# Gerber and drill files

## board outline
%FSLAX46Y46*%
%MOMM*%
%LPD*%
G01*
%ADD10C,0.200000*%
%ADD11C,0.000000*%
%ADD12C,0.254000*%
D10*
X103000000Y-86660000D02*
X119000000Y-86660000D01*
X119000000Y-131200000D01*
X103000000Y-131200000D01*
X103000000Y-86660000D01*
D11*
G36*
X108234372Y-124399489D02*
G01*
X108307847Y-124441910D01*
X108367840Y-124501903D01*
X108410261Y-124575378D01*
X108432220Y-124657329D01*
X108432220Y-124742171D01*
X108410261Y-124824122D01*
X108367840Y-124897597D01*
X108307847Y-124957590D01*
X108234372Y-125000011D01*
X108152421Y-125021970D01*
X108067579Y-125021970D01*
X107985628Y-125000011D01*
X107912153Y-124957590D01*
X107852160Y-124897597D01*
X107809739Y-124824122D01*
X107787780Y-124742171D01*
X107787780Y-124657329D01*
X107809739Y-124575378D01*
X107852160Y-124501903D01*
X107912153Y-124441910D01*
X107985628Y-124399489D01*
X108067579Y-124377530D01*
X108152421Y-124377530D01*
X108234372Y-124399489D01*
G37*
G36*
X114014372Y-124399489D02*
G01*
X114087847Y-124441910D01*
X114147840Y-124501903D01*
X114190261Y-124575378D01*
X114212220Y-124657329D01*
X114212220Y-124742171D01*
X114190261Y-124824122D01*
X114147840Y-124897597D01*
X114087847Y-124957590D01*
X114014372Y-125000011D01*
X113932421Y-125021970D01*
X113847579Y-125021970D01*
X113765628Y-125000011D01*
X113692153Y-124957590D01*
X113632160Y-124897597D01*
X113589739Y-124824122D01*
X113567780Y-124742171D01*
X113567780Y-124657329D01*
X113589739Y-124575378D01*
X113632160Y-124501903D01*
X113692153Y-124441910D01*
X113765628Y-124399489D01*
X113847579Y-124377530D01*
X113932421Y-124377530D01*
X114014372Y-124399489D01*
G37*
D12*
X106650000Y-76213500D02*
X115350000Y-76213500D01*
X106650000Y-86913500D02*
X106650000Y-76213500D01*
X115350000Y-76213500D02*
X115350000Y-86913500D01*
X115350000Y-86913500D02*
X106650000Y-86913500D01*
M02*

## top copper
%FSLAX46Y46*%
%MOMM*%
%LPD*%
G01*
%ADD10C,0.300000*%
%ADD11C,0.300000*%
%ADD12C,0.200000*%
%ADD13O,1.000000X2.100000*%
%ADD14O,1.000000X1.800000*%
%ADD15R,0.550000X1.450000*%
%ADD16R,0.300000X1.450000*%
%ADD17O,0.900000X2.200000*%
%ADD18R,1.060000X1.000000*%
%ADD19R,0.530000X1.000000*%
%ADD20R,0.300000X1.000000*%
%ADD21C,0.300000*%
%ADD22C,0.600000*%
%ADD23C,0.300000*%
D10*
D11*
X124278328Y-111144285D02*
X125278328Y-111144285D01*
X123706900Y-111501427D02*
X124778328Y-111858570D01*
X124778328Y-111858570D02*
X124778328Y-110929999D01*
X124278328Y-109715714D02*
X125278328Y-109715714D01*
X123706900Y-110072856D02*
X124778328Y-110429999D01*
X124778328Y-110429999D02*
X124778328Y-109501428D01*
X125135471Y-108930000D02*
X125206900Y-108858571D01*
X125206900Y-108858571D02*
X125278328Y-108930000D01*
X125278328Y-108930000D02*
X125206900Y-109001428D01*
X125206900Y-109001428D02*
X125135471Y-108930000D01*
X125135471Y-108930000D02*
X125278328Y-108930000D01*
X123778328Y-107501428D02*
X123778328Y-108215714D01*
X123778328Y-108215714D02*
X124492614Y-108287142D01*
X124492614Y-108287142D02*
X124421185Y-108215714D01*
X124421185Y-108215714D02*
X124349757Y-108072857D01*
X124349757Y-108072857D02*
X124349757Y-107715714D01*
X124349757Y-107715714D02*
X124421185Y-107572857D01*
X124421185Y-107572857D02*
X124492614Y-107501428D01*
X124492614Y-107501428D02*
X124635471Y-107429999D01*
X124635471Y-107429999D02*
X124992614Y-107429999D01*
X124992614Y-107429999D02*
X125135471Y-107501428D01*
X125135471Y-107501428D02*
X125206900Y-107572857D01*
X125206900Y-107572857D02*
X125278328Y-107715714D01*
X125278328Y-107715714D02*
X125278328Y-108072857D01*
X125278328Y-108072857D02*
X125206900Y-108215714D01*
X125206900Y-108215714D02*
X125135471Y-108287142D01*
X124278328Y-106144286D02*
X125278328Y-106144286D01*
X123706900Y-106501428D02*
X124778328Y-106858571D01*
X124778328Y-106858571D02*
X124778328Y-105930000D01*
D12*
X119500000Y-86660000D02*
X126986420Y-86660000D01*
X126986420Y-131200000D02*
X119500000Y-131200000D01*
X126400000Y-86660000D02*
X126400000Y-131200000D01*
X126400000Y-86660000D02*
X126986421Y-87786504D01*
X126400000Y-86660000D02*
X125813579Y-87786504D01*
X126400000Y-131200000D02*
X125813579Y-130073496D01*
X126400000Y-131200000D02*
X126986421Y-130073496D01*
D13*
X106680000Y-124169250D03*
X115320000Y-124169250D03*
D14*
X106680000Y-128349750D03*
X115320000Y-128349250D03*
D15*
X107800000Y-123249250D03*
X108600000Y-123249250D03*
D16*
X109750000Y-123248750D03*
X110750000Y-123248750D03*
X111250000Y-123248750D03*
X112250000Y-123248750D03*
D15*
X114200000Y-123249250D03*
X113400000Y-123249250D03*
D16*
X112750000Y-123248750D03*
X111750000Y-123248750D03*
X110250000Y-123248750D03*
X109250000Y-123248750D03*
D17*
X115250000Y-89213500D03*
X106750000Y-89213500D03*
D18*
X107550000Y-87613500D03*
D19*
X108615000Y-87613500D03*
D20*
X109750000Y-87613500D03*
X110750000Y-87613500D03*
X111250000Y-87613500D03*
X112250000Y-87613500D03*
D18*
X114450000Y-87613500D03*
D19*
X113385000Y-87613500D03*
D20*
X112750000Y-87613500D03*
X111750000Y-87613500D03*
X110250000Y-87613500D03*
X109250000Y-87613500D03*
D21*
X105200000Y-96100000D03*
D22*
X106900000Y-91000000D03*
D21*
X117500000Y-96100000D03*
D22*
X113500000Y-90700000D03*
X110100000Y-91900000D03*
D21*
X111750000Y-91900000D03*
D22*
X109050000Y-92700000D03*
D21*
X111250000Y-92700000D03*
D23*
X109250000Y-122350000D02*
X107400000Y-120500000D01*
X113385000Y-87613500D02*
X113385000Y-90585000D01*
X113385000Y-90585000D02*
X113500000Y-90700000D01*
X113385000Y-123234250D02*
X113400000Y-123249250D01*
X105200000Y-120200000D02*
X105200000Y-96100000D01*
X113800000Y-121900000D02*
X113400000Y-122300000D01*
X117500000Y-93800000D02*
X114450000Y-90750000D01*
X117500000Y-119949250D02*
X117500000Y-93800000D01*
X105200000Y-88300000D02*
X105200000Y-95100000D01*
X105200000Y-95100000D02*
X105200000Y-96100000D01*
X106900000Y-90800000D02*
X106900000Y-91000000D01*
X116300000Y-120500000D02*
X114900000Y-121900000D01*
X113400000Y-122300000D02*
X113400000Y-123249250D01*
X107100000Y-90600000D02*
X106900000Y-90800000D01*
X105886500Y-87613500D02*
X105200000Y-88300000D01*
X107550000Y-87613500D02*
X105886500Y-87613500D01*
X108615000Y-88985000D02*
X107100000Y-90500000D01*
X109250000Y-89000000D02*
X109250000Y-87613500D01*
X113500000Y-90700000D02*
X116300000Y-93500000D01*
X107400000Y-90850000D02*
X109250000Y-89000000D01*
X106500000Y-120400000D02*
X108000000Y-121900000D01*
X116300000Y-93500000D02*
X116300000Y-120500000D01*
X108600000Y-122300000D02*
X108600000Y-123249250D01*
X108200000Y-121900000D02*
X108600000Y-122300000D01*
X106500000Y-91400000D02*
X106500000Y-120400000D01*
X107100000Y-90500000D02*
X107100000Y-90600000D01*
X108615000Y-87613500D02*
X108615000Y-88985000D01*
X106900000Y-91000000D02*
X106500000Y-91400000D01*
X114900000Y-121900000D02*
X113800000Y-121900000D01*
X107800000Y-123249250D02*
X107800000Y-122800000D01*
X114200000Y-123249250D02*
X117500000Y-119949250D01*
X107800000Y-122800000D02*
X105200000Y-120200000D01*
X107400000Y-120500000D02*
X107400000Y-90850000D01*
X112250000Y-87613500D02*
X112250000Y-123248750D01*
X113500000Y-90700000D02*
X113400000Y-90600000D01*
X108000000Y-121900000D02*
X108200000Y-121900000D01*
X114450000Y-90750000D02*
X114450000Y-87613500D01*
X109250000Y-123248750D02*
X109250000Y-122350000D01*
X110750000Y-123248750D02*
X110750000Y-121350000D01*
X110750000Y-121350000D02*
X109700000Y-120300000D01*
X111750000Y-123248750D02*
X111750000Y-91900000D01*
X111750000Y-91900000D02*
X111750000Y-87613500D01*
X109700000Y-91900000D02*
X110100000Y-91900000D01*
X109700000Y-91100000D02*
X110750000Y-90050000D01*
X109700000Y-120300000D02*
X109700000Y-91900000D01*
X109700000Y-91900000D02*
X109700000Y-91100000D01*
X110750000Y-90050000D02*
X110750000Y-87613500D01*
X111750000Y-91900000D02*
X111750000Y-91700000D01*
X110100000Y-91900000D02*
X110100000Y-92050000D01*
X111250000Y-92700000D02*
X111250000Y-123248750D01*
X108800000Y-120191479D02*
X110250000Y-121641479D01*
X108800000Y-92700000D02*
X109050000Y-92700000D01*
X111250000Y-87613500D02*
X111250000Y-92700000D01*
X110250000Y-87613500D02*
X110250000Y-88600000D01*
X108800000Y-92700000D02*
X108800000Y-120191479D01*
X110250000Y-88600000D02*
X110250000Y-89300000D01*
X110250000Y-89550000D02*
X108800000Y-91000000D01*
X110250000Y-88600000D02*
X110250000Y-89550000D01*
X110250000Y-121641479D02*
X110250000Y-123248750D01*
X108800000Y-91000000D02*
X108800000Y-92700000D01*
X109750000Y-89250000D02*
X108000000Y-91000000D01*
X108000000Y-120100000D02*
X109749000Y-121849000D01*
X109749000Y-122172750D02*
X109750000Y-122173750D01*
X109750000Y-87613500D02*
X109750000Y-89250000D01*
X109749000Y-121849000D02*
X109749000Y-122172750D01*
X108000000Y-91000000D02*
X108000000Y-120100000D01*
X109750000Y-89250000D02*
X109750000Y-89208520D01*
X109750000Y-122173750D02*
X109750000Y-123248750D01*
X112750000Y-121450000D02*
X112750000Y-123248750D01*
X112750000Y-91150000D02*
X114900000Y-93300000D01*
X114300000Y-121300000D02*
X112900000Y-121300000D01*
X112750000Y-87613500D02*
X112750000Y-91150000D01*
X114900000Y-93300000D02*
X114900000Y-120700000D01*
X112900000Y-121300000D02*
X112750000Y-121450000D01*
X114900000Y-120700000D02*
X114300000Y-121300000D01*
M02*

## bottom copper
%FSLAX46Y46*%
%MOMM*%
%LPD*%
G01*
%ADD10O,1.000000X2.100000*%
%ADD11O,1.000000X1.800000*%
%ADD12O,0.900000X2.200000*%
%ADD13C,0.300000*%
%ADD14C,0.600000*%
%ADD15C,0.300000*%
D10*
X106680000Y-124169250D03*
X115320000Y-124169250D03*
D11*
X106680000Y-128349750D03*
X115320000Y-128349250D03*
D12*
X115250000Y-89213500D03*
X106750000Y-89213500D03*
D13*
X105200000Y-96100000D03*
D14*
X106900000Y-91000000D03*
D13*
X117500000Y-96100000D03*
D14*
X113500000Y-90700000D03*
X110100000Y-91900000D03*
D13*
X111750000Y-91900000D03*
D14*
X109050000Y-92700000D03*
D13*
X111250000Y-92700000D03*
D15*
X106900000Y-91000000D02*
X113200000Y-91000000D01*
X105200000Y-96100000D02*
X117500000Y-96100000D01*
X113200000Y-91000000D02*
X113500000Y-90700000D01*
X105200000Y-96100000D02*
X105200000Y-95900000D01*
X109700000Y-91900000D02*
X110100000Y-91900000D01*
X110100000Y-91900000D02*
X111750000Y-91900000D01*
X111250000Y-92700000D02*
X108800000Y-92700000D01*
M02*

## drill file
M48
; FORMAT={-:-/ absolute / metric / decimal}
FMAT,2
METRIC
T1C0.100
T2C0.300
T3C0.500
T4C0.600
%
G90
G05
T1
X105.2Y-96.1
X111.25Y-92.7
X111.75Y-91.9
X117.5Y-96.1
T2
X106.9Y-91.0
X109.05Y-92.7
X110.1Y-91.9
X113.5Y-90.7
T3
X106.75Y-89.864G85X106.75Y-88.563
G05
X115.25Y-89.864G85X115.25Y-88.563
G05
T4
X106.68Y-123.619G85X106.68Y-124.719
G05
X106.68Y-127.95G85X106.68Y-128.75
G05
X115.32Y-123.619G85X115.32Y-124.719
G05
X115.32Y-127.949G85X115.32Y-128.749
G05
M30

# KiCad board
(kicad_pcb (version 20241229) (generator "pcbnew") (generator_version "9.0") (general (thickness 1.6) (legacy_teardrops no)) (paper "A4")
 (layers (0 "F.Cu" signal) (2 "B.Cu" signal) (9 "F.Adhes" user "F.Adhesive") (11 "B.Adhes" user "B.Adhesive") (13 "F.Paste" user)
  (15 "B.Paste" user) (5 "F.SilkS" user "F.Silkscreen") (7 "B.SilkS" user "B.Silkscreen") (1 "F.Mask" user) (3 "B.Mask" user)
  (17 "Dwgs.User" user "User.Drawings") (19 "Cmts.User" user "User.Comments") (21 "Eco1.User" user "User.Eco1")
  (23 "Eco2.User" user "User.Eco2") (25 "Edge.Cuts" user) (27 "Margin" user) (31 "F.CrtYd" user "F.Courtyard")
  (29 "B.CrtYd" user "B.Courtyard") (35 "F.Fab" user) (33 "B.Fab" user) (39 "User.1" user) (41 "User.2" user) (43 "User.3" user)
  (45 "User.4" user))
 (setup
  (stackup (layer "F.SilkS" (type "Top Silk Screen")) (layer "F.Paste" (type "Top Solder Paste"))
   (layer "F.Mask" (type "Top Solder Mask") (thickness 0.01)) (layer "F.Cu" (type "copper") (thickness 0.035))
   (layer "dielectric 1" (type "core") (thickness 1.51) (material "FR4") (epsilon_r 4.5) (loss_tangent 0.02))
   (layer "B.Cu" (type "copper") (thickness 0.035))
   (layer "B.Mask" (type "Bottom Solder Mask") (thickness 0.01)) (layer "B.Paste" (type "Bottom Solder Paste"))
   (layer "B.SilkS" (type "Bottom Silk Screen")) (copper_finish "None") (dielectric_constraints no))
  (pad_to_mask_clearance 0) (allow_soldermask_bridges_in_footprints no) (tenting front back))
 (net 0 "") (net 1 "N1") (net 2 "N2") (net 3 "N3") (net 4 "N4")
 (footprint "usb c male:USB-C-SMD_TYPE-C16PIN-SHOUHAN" (layer "F.Cu") (at 111 125.79925)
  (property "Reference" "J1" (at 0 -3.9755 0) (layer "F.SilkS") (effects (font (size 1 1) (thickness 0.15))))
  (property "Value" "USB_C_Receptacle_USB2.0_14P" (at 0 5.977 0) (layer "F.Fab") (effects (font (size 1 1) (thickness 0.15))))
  (fp_poly
   (pts (xy -2.56778 -1.141921) (xy -2.589739 -1.223872) (xy -2.63216 -1.297347) (xy -2.692153 -1.35734) (xy -2.765628 -1.399761)
    (xy -2.847579 -1.42172) (xy -2.932421 -1.42172) (xy -3.014372 -1.399761) (xy -3.087847 -1.35734) (xy -3.14784 -1.297347)
    (xy -3.190261 -1.223872) (xy -3.21222 -1.141921) (xy -3.21222 -1.057079) (xy -3.190261 -0.975128) (xy -3.14784 -0.901653)
    (xy -3.087847 -0.84166) (xy -3.014372 -0.799239) (xy -2.932421 -0.77728) (xy -2.847579 -0.77728) (xy -2.765628 -0.799239)
    (xy -2.692153 -0.84166) (xy -2.63216 -0.901653) (xy -2.589739 -0.975128) (xy -2.56778 -1.057079))
   (stroke (width 0) (type default)) (fill yes) (layer "Edge.Cuts"))
  (fp_poly
   (pts (xy 3.21222 -1.141921) (xy 3.190261 -1.223872) (xy 3.14784 -1.297347) (xy 3.087847 -1.35734) (xy 3.014372 -1.399761)
    (xy 2.932421 -1.42172) (xy 2.847579 -1.42172) (xy 2.765628 -1.399761) (xy 2.692153 -1.35734) (xy 2.63216 -1.297347)
    (xy 2.589739 -1.223872) (xy 2.56778 -1.141921) (xy 2.56778 -1.057079) (xy 2.589739 -0.975128) (xy 2.63216 -0.901653)
    (xy 2.692153 -0.84166) (xy 2.765628 -0.799239) (xy 2.847579 -0.77728) (xy 2.932421 -0.77728) (xy 3.014372 -0.799239)
    (xy 3.087847 -0.84166) (xy 3.14784 -0.901653) (xy 3.190261 -0.975128) (xy 3.21222 -1.057079))
   (stroke (width 0) (type default)) (fill yes) (layer "Edge.Cuts"))
  (pad "1" thru_hole oval (at -4.32 -1.63) (size 1 2.1) (drill oval 0.6 1.7) (layers "*.Cu" "*.Mask") (remove_unused_layers no))
  (pad "2" thru_hole oval (at 4.32 -1.63) (size 1 2.1) (drill oval 0.6 1.7) (layers "*.Cu" "*.Mask") (remove_unused_layers no))
  (pad "3" thru_hole oval (at -4.32 2.5505) (size 1 1.8) (drill oval 0.6 1.4) (layers "*.Cu" "*.Mask") (remove_unused_layers no))
  (pad "4" thru_hole oval (at 4.32 2.55) (size 1 1.8) (drill oval 0.6 1.4) (layers "*.Cu" "*.Mask") (remove_unused_layers no))
  (pad "A1B12" smd rect (at -3.2 -2.55) (size 0.55 1.45) (layers "F.Cu" "F.Mask" "F.Paste"))
  (pad "A4B9" smd rect (at -2.4 -2.55) (size 0.55 1.45) (layers "F.Cu" "F.Mask" "F.Paste"))
  (pad "A5" smd rect (at -1.25 -2.5505) (size 0.3 1.45) (layers "F.Cu" "F.Mask" "F.Paste") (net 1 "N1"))
  (pad "A6" smd rect (at -0.25 -2.5505) (size 0.3 1.45) (layers "F.Cu" "F.Mask" "F.Paste") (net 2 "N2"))
  (pad "A7" smd rect (at 0.25 -2.5505) (size 0.3 1.45) (layers "F.Cu" "F.Mask" "F.Paste") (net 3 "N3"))
  (pad "A8" smd rect (at 1.25 -2.5505) (size 0.3 1.45) (layers "F.Cu" "F.Mask" "F.Paste"))
  (pad "B1A12" smd rect (at 3.2 -2.55) (size 0.55 1.45) (layers "F.Cu" "F.Mask" "F.Paste"))
  (pad "B4A9" smd rect (at 2.4 -2.55) (size 0.55 1.45) (layers "F.Cu" "F.Mask" "F.Paste"))
  (pad "B5" smd rect (at 1.75 -2.5505) (size 0.3 1.45) (layers "F.Cu" "F.Mask" "F.Paste") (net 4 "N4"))
  (pad "B6" smd rect (at 0.75 -2.5505) (size 0.3 1.45) (layers "F.Cu" "F.Mask" "F.Paste") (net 2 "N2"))
  (pad "B7" smd rect (at -0.75 -2.5505) (size 0.3 1.45) (layers "F.Cu" "F.Mask" "F.Paste") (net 3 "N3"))
  (pad "B8" smd rect (at -1.75 -2.5505) (size 0.3 1.45) (layers "F.Cu" "F.Mask" "F.Paste")))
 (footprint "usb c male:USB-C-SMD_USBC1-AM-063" (layer "F.Cu") (at 111 88.4135 180)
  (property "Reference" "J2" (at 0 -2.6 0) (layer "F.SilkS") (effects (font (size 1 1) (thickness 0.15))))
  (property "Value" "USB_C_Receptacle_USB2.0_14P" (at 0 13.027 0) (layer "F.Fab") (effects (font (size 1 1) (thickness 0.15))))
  (fp_line (start 4.35 12.2) (end -4.35 12.2) (stroke (width 0.254) (type default)) (layer "Edge.Cuts"))
  (fp_line (start 4.35 1.5) (end 4.35 12.2) (stroke (width 0.254) (type default)) (layer "Edge.Cuts"))
  (fp_line (start -4.35 12.2) (end -4.35 1.5) (stroke (width 0.254) (type default)) (layer "Edge.Cuts"))
  (fp_line (start -4.35 1.5) (end 4.35 1.5) (stroke (width 0.254) (type default)) (layer "Edge.Cuts"))
  (pad "1" thru_hole oval (at -4.25 -0.8 180) (size 0.9 2.2) (drill oval 0.5 1.8) (layers "*.Cu" "*.Mask") (remove_unused_layers no))
  (pad "2" thru_hole oval (at 4.25 -0.8 180) (size 0.9 2.2) (drill oval 0.5 1.8) (layers "*.Cu" "*.Mask") (remove_unused_layers no))
  (pad "A1B12" smd rect (at 3.45 0.8) (size 1.06 1) (layers "F.Cu" "F.Mask" "F.Paste"))
  (pad "A4B9" smd rect (at 2.385 0.8) (size 0.53 1) (layers "F.Cu" "F.Mask" "F.Paste"))
  (pad "A5" smd rect (at 1.25 0.8) (size 0.3 1) (layers "F.Cu" "F.Mask" "F.Paste") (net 1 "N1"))
  (pad "A6" smd rect (at 0.25 0.8 180) (size 0.3 1) (layers "F.Cu" "F.Mask" "F.Paste") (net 2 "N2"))
  (pad "A7" smd rect (at -0.25 0.8) (size 0.3 1) (layers "F.Cu" "F.Mask" "F.Paste") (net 3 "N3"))
  (pad "A8" smd rect (at -1.25 0.8) (size 0.3 1) (layers "F.Cu" "F.Mask" "F.Paste"))
  (pad "B1A12" smd rect (at -3.45 0.8) (size 1.06 1) (layers "F.Cu" "F.Mask" "F.Paste"))
  (pad "B4A9" smd rect (at -2.385 0.8) (size 0.53 1) (layers "F.Cu" "F.Mask" "F.Paste"))
  (pad "B5" smd rect (at -1.75 0.8) (size 0.3 1) (layers "F.Cu" "F.Mask" "F.Paste") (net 4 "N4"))
  (pad "B6" smd rect (at -0.75 0.8 180) (size 0.3 1) (layers "F.Cu" "F.Mask" "F.Paste") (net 2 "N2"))
  (pad "B7" smd rect (at 0.75 0.8) (size 0.3 1) (layers "F.Cu" "F.Mask" "F.Paste") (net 3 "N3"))
  (pad "B8" smd rect (at 1.75 0.8) (size 0.3 1) (layers "F.Cu" "F.Mask" "F.Paste")))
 (gr_rect (start 103 86.66) (end 119 131.2) (stroke (width 0.2) (type solid)) (fill no) (layer "Edge.Cuts"))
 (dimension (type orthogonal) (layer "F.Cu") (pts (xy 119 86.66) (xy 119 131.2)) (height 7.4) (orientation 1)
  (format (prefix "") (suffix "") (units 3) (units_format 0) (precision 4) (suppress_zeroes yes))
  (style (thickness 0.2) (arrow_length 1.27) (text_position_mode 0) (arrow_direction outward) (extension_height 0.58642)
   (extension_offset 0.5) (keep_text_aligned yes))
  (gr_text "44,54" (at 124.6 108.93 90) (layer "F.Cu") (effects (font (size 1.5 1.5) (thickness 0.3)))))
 (segment (start 109.25 122.35) (end 107.4 120.5) (width 0.3) (layer "F.Cu") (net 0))
 (segment (start 113.385 87.6135) (end 113.385 90.585) (width 0.3) (layer "F.Cu") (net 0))
 (segment (start 113.385 90.585) (end 113.5 90.7) (width 0.3) (layer "F.Cu") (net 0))
 (segment (start 113.385 123.23425) (end 113.4 123.24925) (width 0.3) (layer "F.Cu") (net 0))
 (segment (start 105.2 120.2) (end 105.2 96.1) (width 0.3) (layer "F.Cu") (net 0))
 (segment (start 113.8 121.9) (end 113.4 122.3) (width 0.3) (layer "F.Cu") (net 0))
 (segment (start 117.5 93.8) (end 114.45 90.75) (width 0.3) (layer "F.Cu") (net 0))
 (segment (start 117.5 119.94925) (end 117.5 93.8) (width 0.3) (layer "F.Cu") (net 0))
 (segment (start 105.2 88.3) (end 105.2 95.1) (width 0.3) (layer "F.Cu") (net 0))
 (segment (start 105.2 95.1) (end 105.2 96.1) (width 0.3) (layer "F.Cu") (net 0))
 (segment (start 106.9 90.8) (end 106.9 91) (width 0.3) (layer "F.Cu") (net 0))
 (segment (start 116.3 120.5) (end 114.9 121.9) (width 0.3) (layer "F.Cu") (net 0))
 (segment (start 113.4 122.3) (end 113.4 123.24925) (width 0.3) (layer "F.Cu") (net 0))
 (segment (start 107.1 90.6) (end 106.9 90.8) (width 0.3) (layer "F.Cu") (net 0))
 (segment (start 105.8865 87.6135) (end 105.2 88.3) (width 0.3) (layer "F.Cu") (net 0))
 (segment (start 107.55 87.6135) (end 105.8865 87.6135) (width 0.3) (layer "F.Cu") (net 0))
 (segment (start 108.615 88.985) (end 107.1 90.5) (width 0.3) (layer "F.Cu") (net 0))
 (segment (start 109.25 89) (end 109.25 87.6135) (width 0.3) (layer "F.Cu") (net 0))
 (segment (start 113.5 90.7) (end 116.3 93.5) (width 0.3) (layer "F.Cu") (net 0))
 (segment (start 107.4 90.85) (end 109.25 89) (width 0.3) (layer "F.Cu") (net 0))
 (segment (start 106.5 120.4) (end 108 121.9) (width 0.3) (layer "F.Cu") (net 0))
 (segment (start 116.3 93.5) (end 116.3 120.5) (width 0.3) (layer "F.Cu") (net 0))
 (segment (start 108.6 122.3) (end 108.6 123.24925) (width 0.3) (layer "F.Cu") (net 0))
 (segment (start 108.2 121.9) (end 108.6 122.3) (width 0.3) (layer "F.Cu") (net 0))
 (segment (start 106.5 91.4) (end 106.5 120.4) (width 0.3) (layer "F.Cu") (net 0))
 (segment (start 107.1 90.5) (end 107.1 90.6) (width 0.3) (layer "F.Cu") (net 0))
 (segment (start 108.615 87.6135) (end 108.615 88.985) (width 0.3) (layer "F.Cu") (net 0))
 (segment (start 106.9 91) (end 106.5 91.4) (width 0.3) (layer "F.Cu") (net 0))
 (segment (start 114.9 121.9) (end 113.8 121.9) (width 0.3) (layer "F.Cu") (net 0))
 (segment (start 107.8 123.24925) (end 107.8 122.8) (width 0.3) (layer "F.Cu") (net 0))
 (segment (start 114.2 123.24925) (end 117.5 119.94925) (width 0.3) (layer "F.Cu") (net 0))
 (segment (start 107.8 122.8) (end 105.2 120.2) (width 0.3) (layer "F.Cu") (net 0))
 (segment (start 107.4 120.5) (end 107.4 90.85) (width 0.3) (layer "F.Cu") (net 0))
 (segment (start 112.25 87.6135) (end 112.25 123.24875) (width 0.3) (layer "F.Cu") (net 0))
 (segment (start 113.5 90.7) (end 113.4 90.6) (width 0.3) (layer "F.Cu") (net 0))
 (segment (start 108 121.9) (end 108.2 121.9) (width 0.3) (layer "F.Cu") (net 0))
 (segment (start 114.45 90.75) (end 114.45 87.6135) (width 0.3) (layer "F.Cu") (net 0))
 (segment (start 109.25 123.24875) (end 109.25 122.35) (width 0.3) (layer "F.Cu") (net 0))
 (via micro (at 105.2 96.1) (size 0.3) (drill 0.1) (layers "F.Cu" "B.Cu") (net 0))
 (via blind (at 106.9 91) (size 0.6) (drill 0.3) (layers "F.Cu" "B.Cu") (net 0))
 (via micro (at 117.5 96.1) (size 0.3) (drill 0.1) (layers "F.Cu" "B.Cu") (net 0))
 (via blind (at 113.5 90.7) (size 0.6) (drill 0.3) (layers "F.Cu" "B.Cu") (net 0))
 (segment (start 106.9 91) (end 113.2 91) (width 0.3) (layer "B.Cu") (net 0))
 (segment (start 105.2 96.1) (end 117.5 96.1) (width 0.3) (layer "B.Cu") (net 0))
 (segment (start 113.2 91) (end 113.5 90.7) (width 0.3) (layer "B.Cu") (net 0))
 (segment (start 105.2 96.1) (end 105.2 95.9) (width 0.3) (layer "B.Cu") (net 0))
 (segment (start 110.75 123.24875) (end 110.75 121.35) (width 0.3) (layer "F.Cu") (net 2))
 (segment (start 110.75 121.35) (end 109.7 120.3) (width 0.3) (layer "F.Cu") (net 2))
 (segment (start 111.75 123.24875) (end 111.75 91.9) (width 0.3) (layer "F.Cu") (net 2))
 (segment (start 111.75 91.9) (end 111.75 87.6135) (width 0.3) (layer "F.Cu") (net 2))
 (segment (start 109.7 91.9) (end 110.1 91.9) (width 0.3) (layer "F.Cu") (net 2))
 (segment (start 109.7 91.1) (end 110.75 90.05) (width 0.3) (layer "F.Cu") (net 2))
 (segment (start 109.7 120.3) (end 109.7 91.9) (width 0.3) (layer "F.Cu") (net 2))
 (segment (start 109.7 91.9) (end 109.7 91.1) (width 0.3) (layer "F.Cu") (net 2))
 (segment (start 110.75 90.05) (end 110.75 87.6135) (width 0.3) (layer "F.Cu") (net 2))
 (segment (start 111.75 91.9) (end 111.75 91.7) (width 0.3) (layer "F.Cu") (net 2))
 (segment (start 110.1 91.9) (end 110.1 92.05) (width 0.3) (layer "F.Cu") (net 2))
 (via blind (at 110.1 91.9) (size 0.6) (drill 0.3) (layers "F.Cu" "B.Cu") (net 2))
 (via micro (at 111.75 91.9) (size 0.3) (drill 0.1) (layers "F.Cu" "B.Cu") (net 2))
 (segment (start 109.7 91.9) (end 110.1 91.9) (width 0.3) (layer "B.Cu") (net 2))
 (segment (start 110.1 91.9) (end 111.75 91.9) (width 0.3) (layer "B.Cu") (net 2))
 (segment (start 111.25 92.7) (end 111.25 123.24875) (width 0.3) (layer "F.Cu") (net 3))
 (segment (start 108.8 120.191479) (end 110.25 121.641479) (width 0.3) (layer "F.Cu") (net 3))
 (segment (start 108.8 92.7) (end 109.05 92.7) (width 0.3) (layer "F.Cu") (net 3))
 (segment (start 111.25 87.6135) (end 111.25 92.7) (width 0.3) (layer "F.Cu") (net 3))
 (segment (start 110.25 87.6135) (end 110.25 88.6) (width 0.3) (layer "F.Cu") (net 3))
 (segment (start 108.8 92.7) (end 108.8 120.191479) (width 0.3) (layer "F.Cu") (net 3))
 (segment (start 110.25 88.6) (end 110.25 89.3) (width 0.3) (layer "F.Cu") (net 3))
 (segment (start 110.25 89.55) (end 108.8 91) (width 0.3) (layer "F.Cu") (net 3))
 (segment (start 110.25 88.6) (end 110.25 89.55) (width 0.3) (layer "F.Cu") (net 3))
 (segment (start 110.25 121.641479) (end 110.25 123.24875) (width 0.3) (layer "F.Cu") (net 3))
 (segment (start 108.8 91) (end 108.8 92.7) (width 0.3) (layer "F.Cu") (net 3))
 (via blind (at 109.05 92.7) (size 0.6) (drill 0.3) (layers "F.Cu" "B.Cu") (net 3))
 (via micro (at 111.25 92.7) (size 0.3) (drill 0.1) (layers "F.Cu" "B.Cu") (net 3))
 (segment (start 111.25 92.7) (end 108.8 92.7) (width 0.3) (layer "B.Cu") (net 3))
 (segment (start 109.75 89.25) (end 108 91) (width 0.3) (layer "F.Cu") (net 1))
 (segment (start 108 120.1) (end 109.749 121.849) (width 0.3) (layer "F.Cu") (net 1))
 (segment (start 109.749 122.17275) (end 109.75 122.17375) (width 0.3) (layer "F.Cu") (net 1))
 (segment (start 109.75 87.6135) (end 109.75 89.25) (width 0.3) (layer "F.Cu") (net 1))
 (segment (start 109.749 121.849) (end 109.749 122.17275) (width 0.3) (layer "F.Cu") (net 1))
 (segment (start 108 91) (end 108 120.1) (width 0.3) (layer "F.Cu") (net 1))
 (segment (start 109.75 89.25) (end 109.75 89.20852) (width 0.3) (layer "F.Cu") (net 1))
 (segment (start 109.75 122.17375) (end 109.75 123.24875) (width 0.3) (layer "F.Cu") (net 1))
 (segment (start 112.75 121.45) (end 112.75 123.24875) (width 0.3) (layer "F.Cu") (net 4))
 (segment (start 112.75 91.15) (end 114.9 93.3) (width 0.3) (layer "F.Cu") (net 4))
 (segment (start 114.3 121.3) (end 112.9 121.3) (width 0.3) (layer "F.Cu") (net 4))
 (segment (start 112.75 87.6135) (end 112.75 91.15) (width 0.3) (layer "F.Cu") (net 4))
 (segment (start 114.9 93.3) (end 114.9 120.7) (width 0.3) (layer "F.Cu") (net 4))
 (segment (start 112.9 121.3) (end 112.75 121.45) (width 0.3) (layer "F.Cu") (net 4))
 (segment (start 114.9 120.7) (end 114.3 121.3) (width 0.3) (layer "F.Cu") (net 4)))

